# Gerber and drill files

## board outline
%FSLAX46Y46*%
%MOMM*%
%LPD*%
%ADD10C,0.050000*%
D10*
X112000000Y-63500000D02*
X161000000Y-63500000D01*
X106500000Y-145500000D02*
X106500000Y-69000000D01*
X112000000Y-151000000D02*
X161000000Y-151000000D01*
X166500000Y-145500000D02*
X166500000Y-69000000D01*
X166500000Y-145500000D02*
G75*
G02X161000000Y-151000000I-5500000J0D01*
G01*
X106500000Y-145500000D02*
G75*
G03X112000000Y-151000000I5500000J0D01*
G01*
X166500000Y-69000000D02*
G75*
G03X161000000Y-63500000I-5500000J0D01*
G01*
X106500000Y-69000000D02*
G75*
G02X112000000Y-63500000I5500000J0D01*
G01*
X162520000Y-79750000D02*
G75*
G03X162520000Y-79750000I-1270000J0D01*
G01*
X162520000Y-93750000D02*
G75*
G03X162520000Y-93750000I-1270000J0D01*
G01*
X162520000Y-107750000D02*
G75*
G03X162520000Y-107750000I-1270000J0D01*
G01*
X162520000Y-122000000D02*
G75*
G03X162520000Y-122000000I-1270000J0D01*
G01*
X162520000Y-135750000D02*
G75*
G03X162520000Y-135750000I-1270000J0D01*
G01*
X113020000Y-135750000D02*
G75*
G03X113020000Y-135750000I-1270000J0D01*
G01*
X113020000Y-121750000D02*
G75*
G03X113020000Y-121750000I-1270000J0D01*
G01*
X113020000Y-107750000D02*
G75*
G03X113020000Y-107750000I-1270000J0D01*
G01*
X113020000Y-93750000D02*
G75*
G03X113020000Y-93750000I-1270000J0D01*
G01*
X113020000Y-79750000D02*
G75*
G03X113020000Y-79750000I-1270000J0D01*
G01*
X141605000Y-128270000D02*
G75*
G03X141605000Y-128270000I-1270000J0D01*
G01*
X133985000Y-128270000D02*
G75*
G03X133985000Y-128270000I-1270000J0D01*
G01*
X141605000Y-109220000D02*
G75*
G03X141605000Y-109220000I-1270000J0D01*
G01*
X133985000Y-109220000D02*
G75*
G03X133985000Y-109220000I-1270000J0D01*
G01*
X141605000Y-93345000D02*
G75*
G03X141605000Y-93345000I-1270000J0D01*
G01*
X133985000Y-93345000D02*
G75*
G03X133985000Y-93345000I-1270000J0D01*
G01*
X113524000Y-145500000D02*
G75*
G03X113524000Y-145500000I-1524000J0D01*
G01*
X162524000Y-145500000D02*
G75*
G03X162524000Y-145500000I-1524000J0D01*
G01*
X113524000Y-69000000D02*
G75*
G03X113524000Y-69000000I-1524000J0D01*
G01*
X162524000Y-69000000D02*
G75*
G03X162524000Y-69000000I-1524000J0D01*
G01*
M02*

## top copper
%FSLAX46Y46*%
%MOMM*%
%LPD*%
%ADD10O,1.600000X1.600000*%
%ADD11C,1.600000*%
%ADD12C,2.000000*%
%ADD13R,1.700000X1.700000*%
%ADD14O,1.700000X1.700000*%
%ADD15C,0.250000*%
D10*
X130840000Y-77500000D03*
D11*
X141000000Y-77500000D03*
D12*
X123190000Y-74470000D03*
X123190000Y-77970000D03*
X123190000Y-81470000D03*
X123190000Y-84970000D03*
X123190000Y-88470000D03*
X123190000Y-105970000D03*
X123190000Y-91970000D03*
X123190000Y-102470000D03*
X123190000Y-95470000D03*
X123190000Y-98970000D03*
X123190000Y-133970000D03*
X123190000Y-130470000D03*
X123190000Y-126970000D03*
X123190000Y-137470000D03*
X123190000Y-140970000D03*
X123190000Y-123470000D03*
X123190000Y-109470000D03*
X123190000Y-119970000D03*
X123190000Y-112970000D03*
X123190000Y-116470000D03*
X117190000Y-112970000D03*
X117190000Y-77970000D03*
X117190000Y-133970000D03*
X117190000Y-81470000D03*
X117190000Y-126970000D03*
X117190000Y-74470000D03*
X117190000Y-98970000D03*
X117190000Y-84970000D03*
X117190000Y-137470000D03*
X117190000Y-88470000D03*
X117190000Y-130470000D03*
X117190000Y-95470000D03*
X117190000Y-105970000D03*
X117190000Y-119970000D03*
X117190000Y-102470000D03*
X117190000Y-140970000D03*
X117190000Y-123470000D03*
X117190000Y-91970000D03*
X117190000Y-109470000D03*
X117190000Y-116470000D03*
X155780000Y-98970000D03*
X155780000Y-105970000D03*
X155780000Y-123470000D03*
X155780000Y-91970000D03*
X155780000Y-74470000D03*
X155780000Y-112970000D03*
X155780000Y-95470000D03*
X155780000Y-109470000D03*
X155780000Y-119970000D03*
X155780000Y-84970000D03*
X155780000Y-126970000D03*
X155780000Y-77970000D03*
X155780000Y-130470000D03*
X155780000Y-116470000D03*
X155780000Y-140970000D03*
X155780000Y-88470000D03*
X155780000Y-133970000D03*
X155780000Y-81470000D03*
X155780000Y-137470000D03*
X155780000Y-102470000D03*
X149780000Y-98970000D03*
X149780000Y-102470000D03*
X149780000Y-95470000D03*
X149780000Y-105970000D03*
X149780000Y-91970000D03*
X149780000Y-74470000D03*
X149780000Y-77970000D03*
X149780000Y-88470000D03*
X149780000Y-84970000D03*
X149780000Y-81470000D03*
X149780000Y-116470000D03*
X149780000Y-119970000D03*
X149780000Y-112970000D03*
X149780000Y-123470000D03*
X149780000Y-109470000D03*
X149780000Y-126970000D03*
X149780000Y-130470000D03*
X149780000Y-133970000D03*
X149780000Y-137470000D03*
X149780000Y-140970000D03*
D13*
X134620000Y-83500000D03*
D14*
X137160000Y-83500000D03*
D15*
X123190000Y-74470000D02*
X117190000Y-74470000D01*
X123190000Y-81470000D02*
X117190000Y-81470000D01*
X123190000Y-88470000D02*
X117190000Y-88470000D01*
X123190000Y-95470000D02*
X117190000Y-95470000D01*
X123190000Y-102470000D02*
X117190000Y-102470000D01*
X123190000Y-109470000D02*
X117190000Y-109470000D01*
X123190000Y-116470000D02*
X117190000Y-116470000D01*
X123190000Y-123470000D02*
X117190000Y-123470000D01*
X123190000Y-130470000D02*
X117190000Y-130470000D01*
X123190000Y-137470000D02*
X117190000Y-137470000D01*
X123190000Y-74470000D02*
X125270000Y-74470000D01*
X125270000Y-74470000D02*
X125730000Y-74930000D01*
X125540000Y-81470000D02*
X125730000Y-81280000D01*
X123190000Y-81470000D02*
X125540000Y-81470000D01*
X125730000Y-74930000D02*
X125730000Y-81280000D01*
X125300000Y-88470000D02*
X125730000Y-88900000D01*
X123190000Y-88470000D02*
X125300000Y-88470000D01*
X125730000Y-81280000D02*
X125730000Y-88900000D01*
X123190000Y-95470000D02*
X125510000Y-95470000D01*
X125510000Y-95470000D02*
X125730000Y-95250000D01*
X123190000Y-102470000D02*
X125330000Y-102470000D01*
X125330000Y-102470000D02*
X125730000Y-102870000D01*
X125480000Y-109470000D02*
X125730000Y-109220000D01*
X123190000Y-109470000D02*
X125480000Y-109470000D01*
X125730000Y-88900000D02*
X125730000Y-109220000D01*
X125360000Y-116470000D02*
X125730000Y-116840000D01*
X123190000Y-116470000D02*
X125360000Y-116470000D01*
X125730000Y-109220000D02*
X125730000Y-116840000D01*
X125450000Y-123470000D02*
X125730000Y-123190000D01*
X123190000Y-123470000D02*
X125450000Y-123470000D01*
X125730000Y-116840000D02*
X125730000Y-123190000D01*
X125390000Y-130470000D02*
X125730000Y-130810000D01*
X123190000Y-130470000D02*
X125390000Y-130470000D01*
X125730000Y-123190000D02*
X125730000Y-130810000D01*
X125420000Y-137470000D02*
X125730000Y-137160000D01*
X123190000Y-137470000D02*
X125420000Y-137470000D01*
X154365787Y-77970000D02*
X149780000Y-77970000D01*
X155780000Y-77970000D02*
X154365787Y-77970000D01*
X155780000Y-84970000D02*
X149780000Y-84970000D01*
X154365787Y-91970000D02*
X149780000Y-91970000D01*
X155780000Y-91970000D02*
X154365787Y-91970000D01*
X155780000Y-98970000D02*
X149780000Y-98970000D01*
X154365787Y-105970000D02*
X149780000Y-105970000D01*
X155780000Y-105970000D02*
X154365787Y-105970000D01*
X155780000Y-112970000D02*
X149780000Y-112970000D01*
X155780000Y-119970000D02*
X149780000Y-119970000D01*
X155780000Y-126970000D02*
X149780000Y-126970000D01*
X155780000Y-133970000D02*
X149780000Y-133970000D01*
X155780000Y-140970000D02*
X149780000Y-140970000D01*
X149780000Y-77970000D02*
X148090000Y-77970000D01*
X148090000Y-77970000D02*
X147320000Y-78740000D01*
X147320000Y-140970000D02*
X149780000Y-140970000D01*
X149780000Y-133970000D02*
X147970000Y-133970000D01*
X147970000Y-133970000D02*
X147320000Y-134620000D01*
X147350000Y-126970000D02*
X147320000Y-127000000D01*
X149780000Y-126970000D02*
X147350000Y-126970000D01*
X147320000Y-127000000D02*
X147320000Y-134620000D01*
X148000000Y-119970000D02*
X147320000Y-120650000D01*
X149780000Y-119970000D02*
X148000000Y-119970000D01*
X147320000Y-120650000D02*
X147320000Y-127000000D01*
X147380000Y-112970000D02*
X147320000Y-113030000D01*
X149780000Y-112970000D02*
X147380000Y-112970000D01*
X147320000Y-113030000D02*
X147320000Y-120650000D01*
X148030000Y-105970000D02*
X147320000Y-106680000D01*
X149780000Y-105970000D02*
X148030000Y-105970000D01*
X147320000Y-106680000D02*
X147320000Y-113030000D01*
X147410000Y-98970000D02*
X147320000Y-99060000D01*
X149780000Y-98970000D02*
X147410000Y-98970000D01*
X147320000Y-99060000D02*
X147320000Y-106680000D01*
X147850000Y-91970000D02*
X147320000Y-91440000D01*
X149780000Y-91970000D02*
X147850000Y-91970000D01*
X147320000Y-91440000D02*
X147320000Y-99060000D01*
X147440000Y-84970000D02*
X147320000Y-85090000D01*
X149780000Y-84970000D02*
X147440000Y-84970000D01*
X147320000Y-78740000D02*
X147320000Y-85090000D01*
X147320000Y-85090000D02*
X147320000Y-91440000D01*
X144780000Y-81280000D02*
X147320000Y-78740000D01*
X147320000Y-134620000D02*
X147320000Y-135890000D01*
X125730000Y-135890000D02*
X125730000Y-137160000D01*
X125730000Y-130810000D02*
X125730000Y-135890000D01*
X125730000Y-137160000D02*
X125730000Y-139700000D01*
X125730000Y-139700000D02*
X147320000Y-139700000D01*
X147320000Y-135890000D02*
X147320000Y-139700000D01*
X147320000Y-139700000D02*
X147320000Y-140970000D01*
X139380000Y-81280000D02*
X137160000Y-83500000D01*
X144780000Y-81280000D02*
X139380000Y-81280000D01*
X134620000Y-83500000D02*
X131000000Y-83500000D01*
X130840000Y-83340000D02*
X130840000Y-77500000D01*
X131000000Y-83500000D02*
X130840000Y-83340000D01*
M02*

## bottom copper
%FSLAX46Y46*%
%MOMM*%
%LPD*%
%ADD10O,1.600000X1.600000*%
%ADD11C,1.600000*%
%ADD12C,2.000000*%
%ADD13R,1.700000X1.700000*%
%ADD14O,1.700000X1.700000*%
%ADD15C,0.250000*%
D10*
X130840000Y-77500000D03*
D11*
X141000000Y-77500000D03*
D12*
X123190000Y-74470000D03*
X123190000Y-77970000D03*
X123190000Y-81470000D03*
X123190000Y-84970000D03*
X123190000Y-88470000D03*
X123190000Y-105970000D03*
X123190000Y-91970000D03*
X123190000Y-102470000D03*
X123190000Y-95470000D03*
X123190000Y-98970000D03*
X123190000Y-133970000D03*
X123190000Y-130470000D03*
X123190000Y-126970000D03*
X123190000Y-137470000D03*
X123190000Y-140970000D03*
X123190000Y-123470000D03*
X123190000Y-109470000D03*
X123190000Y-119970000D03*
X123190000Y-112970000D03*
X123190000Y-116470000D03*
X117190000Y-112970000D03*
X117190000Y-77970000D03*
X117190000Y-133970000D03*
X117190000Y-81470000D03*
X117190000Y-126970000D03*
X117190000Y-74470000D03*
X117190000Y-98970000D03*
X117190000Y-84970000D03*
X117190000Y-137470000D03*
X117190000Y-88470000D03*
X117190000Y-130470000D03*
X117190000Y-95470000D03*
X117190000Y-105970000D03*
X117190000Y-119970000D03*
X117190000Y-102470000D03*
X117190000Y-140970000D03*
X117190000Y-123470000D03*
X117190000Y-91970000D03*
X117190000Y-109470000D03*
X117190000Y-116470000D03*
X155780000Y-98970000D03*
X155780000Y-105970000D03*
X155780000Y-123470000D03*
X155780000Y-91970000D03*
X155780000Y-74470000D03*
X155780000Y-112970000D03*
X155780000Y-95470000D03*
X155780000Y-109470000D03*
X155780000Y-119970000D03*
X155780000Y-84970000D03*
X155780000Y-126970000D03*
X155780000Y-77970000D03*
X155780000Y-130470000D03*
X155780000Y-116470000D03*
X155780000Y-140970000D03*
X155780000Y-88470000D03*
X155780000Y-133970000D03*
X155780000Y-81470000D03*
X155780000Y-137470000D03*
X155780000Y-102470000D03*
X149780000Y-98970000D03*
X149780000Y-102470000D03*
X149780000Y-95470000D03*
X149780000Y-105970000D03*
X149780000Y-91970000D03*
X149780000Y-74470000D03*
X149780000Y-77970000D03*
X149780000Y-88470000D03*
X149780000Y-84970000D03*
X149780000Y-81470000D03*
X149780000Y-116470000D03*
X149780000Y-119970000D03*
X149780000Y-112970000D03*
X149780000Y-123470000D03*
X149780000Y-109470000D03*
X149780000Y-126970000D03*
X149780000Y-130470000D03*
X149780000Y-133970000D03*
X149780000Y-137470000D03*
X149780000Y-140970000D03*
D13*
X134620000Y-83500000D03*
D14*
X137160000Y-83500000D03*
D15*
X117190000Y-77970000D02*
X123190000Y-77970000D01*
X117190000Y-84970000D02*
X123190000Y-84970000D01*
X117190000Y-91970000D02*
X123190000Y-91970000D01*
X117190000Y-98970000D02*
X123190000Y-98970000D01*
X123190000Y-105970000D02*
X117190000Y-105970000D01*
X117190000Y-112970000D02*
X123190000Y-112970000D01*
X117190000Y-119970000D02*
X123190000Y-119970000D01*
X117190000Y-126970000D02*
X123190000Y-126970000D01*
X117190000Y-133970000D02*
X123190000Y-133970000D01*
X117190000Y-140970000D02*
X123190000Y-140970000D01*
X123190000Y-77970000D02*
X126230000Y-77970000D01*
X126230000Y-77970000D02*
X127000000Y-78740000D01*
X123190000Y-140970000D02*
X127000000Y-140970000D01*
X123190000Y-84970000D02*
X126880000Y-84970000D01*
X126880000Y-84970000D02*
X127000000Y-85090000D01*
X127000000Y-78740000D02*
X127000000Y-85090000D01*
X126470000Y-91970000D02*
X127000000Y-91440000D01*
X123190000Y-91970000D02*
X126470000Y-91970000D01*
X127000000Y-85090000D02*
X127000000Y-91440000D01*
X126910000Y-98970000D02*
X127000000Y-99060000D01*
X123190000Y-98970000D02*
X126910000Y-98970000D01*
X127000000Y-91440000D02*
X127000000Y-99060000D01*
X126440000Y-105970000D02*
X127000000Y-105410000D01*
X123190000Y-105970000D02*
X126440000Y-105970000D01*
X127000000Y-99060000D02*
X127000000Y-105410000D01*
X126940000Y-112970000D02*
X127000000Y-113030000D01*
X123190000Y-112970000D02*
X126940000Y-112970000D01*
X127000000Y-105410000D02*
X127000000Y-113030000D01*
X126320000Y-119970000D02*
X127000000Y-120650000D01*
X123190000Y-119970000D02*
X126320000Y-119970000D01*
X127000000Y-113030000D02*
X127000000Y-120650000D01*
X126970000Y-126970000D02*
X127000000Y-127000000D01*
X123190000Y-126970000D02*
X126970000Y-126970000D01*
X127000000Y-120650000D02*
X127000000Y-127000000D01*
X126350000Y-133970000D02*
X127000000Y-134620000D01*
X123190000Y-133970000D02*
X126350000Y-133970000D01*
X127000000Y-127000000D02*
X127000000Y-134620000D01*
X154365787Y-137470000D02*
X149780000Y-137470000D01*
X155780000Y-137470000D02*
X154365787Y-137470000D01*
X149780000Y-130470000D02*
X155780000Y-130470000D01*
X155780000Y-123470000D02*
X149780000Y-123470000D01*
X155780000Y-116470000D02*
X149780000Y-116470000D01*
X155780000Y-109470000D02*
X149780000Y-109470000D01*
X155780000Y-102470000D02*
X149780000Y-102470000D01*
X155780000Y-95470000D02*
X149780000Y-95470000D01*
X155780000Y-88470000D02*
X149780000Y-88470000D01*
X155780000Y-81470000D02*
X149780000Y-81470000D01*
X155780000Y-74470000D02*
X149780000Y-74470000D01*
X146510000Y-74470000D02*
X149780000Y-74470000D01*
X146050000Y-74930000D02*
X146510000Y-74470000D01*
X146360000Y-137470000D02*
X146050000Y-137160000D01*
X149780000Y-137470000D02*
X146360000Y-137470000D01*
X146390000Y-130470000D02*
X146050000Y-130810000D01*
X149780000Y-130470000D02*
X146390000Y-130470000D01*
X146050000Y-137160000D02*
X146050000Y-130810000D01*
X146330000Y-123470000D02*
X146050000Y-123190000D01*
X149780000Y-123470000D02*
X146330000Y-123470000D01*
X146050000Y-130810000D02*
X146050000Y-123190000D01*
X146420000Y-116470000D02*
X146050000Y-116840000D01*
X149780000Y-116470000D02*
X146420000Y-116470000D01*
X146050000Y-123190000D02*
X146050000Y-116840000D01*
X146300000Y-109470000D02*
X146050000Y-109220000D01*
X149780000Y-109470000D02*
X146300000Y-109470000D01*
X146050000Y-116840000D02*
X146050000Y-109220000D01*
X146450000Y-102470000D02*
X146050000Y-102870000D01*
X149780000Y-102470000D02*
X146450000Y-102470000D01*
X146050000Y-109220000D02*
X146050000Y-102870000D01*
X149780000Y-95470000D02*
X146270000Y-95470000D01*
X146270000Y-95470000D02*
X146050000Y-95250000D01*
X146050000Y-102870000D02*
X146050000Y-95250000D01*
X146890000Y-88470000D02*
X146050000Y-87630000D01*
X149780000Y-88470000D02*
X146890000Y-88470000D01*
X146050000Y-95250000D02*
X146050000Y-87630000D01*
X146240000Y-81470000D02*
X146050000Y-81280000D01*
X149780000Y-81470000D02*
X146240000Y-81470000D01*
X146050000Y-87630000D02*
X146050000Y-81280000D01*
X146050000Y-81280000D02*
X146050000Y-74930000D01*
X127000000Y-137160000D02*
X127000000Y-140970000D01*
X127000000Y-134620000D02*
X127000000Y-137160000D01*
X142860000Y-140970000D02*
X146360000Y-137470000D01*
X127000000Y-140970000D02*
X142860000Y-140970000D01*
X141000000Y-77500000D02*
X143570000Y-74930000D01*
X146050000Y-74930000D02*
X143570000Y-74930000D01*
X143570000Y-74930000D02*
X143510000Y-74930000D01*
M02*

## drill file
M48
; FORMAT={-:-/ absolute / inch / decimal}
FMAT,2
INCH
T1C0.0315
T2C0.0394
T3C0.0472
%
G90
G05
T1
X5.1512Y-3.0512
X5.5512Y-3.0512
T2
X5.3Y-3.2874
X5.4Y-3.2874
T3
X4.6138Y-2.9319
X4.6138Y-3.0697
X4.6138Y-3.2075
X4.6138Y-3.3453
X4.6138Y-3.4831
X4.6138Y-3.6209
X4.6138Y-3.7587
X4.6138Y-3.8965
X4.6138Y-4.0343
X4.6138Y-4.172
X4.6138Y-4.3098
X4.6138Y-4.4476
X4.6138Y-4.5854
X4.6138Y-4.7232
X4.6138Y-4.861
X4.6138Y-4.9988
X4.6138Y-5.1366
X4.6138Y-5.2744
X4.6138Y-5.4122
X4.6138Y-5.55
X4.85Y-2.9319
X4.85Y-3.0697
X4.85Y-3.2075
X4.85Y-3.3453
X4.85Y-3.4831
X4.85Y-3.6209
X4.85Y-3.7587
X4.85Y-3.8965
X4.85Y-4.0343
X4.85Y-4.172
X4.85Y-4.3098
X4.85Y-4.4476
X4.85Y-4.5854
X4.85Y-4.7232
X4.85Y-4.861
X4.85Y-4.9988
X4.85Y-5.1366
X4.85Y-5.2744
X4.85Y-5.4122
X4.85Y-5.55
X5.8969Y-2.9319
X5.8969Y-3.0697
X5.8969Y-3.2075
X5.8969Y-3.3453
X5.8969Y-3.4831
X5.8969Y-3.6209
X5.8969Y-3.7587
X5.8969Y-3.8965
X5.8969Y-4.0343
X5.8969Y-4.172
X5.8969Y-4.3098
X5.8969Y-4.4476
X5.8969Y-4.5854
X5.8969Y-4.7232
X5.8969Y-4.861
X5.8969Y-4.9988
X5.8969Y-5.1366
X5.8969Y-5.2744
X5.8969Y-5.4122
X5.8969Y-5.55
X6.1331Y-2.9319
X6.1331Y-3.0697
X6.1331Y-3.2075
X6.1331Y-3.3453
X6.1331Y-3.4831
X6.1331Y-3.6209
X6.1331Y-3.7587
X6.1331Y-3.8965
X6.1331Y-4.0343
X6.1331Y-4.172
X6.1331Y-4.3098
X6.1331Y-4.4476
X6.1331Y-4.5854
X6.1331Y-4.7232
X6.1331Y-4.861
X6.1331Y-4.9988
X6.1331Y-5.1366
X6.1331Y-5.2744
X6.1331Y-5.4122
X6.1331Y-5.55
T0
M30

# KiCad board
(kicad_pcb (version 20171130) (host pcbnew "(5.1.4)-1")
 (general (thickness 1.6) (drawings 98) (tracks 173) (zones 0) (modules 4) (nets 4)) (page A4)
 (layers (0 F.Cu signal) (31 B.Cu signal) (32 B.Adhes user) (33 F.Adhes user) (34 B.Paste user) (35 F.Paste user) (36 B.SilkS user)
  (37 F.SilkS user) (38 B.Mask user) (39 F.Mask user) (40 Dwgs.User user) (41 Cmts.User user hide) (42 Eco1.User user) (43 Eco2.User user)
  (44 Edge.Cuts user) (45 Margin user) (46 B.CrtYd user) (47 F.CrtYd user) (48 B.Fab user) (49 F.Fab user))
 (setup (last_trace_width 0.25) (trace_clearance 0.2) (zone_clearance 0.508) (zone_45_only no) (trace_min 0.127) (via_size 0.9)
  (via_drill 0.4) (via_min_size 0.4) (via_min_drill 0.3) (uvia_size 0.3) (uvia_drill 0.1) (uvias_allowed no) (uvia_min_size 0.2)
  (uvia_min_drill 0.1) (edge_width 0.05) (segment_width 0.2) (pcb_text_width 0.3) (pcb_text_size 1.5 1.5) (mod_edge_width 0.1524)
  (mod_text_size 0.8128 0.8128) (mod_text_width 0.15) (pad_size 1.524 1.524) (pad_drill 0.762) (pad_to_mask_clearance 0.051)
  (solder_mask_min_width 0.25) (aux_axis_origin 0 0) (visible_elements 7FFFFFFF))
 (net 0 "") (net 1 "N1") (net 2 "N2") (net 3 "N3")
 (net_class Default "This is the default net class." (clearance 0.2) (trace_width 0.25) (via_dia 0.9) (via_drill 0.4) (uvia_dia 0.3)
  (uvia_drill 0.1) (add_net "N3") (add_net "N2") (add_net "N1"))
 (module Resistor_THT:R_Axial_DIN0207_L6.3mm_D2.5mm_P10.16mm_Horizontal (layer F.Cu) (at 141 77.5 180)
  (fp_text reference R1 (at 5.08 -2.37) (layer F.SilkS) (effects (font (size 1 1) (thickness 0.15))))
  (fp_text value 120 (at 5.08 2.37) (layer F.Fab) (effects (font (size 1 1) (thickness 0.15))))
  (pad 2 thru_hole oval (at 10.16 0 180) (size 1.6 1.6) (drill 0.8) (layers *.Cu *.Mask) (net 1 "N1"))
  (pad 1 thru_hole circle (at 0 0 180) (size 1.6 1.6) (drill 0.8) (layers *.Cu *.Mask) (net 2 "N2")))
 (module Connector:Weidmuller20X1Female (layer F.Cu) (at 128.19 88.97 270)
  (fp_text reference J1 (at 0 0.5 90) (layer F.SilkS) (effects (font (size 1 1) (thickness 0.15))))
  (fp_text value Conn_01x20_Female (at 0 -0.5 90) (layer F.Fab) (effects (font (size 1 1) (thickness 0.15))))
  (pad 1 thru_hole circle (at -14.5 5 270) (size 2 2) (drill 1.2) (layers *.Cu *.Mask) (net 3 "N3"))
  (pad 2 thru_hole circle (at -11 5 270) (size 2 2) (drill 1.2) (layers *.Cu *.Mask) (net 2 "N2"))
  (pad 3 thru_hole circle (at -7.5 5 270) (size 2 2) (drill 1.2) (layers *.Cu *.Mask) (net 3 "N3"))
  (pad 4 thru_hole circle (at -4 5) (size 2 2) (drill 1.2) (layers *.Cu *.Mask) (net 2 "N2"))
  (pad 5 thru_hole circle (at -0.5 5 270) (size 2 2) (drill 1.2) (layers *.Cu *.Mask) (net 3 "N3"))
  (pad 10 thru_hole circle (at 17 5 270) (size 2 2) (drill 1.2) (layers *.Cu *.Mask) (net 2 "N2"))
  (pad 6 thru_hole circle (at 3 5 270) (size 2 2) (drill 1.2) (layers *.Cu *.Mask) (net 2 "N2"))
  (pad 9 thru_hole circle (at 13.5 5 270) (size 2 2) (drill 1.2) (layers *.Cu *.Mask) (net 3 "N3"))
  (pad 7 thru_hole circle (at 6.5 5 270) (size 2 2) (drill 1.2) (layers *.Cu *.Mask) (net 3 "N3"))
  (pad 8 thru_hole circle (at 10 5 270) (size 2 2) (drill 1.2) (layers *.Cu *.Mask) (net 2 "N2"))
  (pad 18 thru_hole circle (at 45 5 270) (size 2 2) (drill 1.2) (layers *.Cu *.Mask) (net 2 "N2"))
  (pad 17 thru_hole circle (at 41.5 5) (size 2 2) (drill 1.2) (layers *.Cu *.Mask) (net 3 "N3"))
  (pad 16 thru_hole circle (at 38 5 270) (size 2 2) (drill 1.2) (layers *.Cu *.Mask) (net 2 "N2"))
  (pad 19 thru_hole circle (at 48.5 5 270) (size 2 2) (drill 1.2) (layers *.Cu *.Mask) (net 3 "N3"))
  (pad 20 thru_hole circle (at 52 5 270) (size 2 2) (drill 1.2) (layers *.Cu *.Mask) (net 2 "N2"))
  (pad 15 thru_hole circle (at 34.5 5 270) (size 2 2) (drill 1.2) (layers *.Cu *.Mask) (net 3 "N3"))
  (pad 11 thru_hole circle (at 20.5 5 270) (size 2 2) (drill 1.2) (layers *.Cu *.Mask) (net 3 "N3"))
  (pad 14 thru_hole circle (at 31 5 270) (size 2 2) (drill 1.2) (layers *.Cu *.Mask) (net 2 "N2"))
  (pad 12 thru_hole circle (at 24 5 270) (size 2 2) (drill 1.2) (layers *.Cu *.Mask) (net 2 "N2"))
  (pad 13 thru_hole circle (at 27.5 5 270) (size 2 2) (drill 1.2) (layers *.Cu *.Mask) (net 3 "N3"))
  (pad 12 thru_hole circle (at 24 11 270) (size 2 2) (drill 1.2) (layers *.Cu *.Mask) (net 2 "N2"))
  (pad 2 thru_hole circle (at -11 11 270) (size 2 2) (drill 1.2) (layers *.Cu *.Mask) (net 2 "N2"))
  (pad 18 thru_hole circle (at 45 11 270) (size 2 2) (drill 1.2) (layers *.Cu *.Mask) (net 2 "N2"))
  (pad 3 thru_hole circle (at -7.5 11 270) (size 2 2) (drill 1.2) (layers *.Cu *.Mask) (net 3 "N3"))
  (pad 16 thru_hole circle (at 38 11 270) (size 2 2) (drill 1.2) (layers *.Cu *.Mask) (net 2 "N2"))
  (pad 1 thru_hole circle (at -14.5 11 270) (size 2 2) (drill 1.2) (layers *.Cu *.Mask) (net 3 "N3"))
  (pad 8 thru_hole circle (at 10 11 270) (size 2 2) (drill 1.2) (layers *.Cu *.Mask) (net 2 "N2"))
  (pad 4 thru_hole circle (at -4 11) (size 2 2) (drill 1.2) (layers *.Cu *.Mask) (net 2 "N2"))
  (pad 19 thru_hole circle (at 48.5 11 270) (size 2 2) (drill 1.2) (layers *.Cu *.Mask) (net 3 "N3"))
  (pad 5 thru_hole circle (at -0.5 11 270) (size 2 2) (drill 1.2) (layers *.Cu *.Mask) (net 3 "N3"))
  (pad 17 thru_hole circle (at 41.5 11) (size 2 2) (drill 1.2) (layers *.Cu *.Mask) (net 3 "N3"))
  (pad 7 thru_hole circle (at 6.5 11 270) (size 2 2) (drill 1.2) (layers *.Cu *.Mask) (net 3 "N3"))
  (pad 10 thru_hole circle (at 17 11 270) (size 2 2) (drill 1.2) (layers *.Cu *.Mask) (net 2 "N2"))
  (pad 14 thru_hole circle (at 31 11 270) (size 2 2) (drill 1.2) (layers *.Cu *.Mask) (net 2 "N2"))
  (pad 9 thru_hole circle (at 13.5 11 270) (size 2 2) (drill 1.2) (layers *.Cu *.Mask) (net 3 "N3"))
  (pad 20 thru_hole circle (at 52 11 270) (size 2 2) (drill 1.2) (layers *.Cu *.Mask) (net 2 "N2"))
  (pad 15 thru_hole circle (at 34.5 11 270) (size 2 2) (drill 1.2) (layers *.Cu *.Mask) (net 3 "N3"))
  (pad 6 thru_hole circle (at 3 11 270) (size 2 2) (drill 1.2) (layers *.Cu *.Mask) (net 2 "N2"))
  (pad 11 thru_hole circle (at 20.5 11 270) (size 2 2) (drill 1.2) (layers *.Cu *.Mask) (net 3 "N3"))
  (pad 13 thru_hole circle (at 27.5 11 270) (size 2 2) (drill 1.2) (layers *.Cu *.Mask) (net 3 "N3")))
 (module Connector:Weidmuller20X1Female (layer F.Cu) (at 144.78 126.47 90)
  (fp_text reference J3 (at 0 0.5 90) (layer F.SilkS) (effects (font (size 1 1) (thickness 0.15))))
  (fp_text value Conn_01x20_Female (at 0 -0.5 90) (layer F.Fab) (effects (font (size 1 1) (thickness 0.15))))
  (pad 13 thru_hole circle (at 27.5 11 90) (size 2 2) (drill 1.2) (layers *.Cu *.Mask) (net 3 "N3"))
  (pad 11 thru_hole circle (at 20.5 11 90) (size 2 2) (drill 1.2) (layers *.Cu *.Mask) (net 3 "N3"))
  (pad 6 thru_hole circle (at 3 11 90) (size 2 2) (drill 1.2) (layers *.Cu *.Mask) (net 2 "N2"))
  (pad 15 thru_hole circle (at 34.5 11 90) (size 2 2) (drill 1.2) (layers *.Cu *.Mask) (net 3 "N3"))
  (pad 20 thru_hole circle (at 52 11 90) (size 2 2) (drill 1.2) (layers *.Cu *.Mask) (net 2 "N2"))
  (pad 9 thru_hole circle (at 13.5 11 90) (size 2 2) (drill 1.2) (layers *.Cu *.Mask) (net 3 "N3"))
  (pad 14 thru_hole circle (at 31 11 90) (size 2 2) (drill 1.2) (layers *.Cu *.Mask) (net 2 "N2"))
  (pad 10 thru_hole circle (at 17 11 90) (size 2 2) (drill 1.2) (layers *.Cu *.Mask) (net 2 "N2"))
  (pad 7 thru_hole circle (at 6.5 11 90) (size 2 2) (drill 1.2) (layers *.Cu *.Mask) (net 3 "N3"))
  (pad 17 thru_hole circle (at 41.5 11 180) (size 2 2) (drill 1.2) (layers *.Cu *.Mask) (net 3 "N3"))
  (pad 5 thru_hole circle (at -0.5 11 90) (size 2 2) (drill 1.2) (layers *.Cu *.Mask) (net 3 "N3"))
  (pad 19 thru_hole circle (at 48.5 11 90) (size 2 2) (drill 1.2) (layers *.Cu *.Mask) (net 3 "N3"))
  (pad 4 thru_hole circle (at -4 11 180) (size 2 2) (drill 1.2) (layers *.Cu *.Mask) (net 2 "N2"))
  (pad 8 thru_hole circle (at 10 11 90) (size 2 2) (drill 1.2) (layers *.Cu *.Mask) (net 2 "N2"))
  (pad 1 thru_hole circle (at -14.5 11 90) (size 2 2) (drill 1.2) (layers *.Cu *.Mask) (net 3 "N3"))
  (pad 16 thru_hole circle (at 38 11 90) (size 2 2) (drill 1.2) (layers *.Cu *.Mask) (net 2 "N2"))
  (pad 3 thru_hole circle (at -7.5 11 90) (size 2 2) (drill 1.2) (layers *.Cu *.Mask) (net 3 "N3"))
  (pad 18 thru_hole circle (at 45 11 90) (size 2 2) (drill 1.2) (layers *.Cu *.Mask) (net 2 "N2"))
  (pad 2 thru_hole circle (at -11 11 90) (size 2 2) (drill 1.2) (layers *.Cu *.Mask) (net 2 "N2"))
  (pad 12 thru_hole circle (at 24 11 90) (size 2 2) (drill 1.2) (layers *.Cu *.Mask) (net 2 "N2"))
  (pad 13 thru_hole circle (at 27.5 5 90) (size 2 2) (drill 1.2) (layers *.Cu *.Mask) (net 3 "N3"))
  (pad 12 thru_hole circle (at 24 5 90) (size 2 2) (drill 1.2) (layers *.Cu *.Mask) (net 2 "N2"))
  (pad 14 thru_hole circle (at 31 5 90) (size 2 2) (drill 1.2) (layers *.Cu *.Mask) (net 2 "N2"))
  (pad 11 thru_hole circle (at 20.5 5 90) (size 2 2) (drill 1.2) (layers *.Cu *.Mask) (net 3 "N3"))
  (pad 15 thru_hole circle (at 34.5 5 90) (size 2 2) (drill 1.2) (layers *.Cu *.Mask) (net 3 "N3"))
  (pad 20 thru_hole circle (at 52 5 90) (size 2 2) (drill 1.2) (layers *.Cu *.Mask) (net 2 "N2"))
  (pad 19 thru_hole circle (at 48.5 5 90) (size 2 2) (drill 1.2) (layers *.Cu *.Mask) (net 3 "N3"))
  (pad 16 thru_hole circle (at 38 5 90) (size 2 2) (drill 1.2) (layers *.Cu *.Mask) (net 2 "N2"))
  (pad 17 thru_hole circle (at 41.5 5 180) (size 2 2) (drill 1.2) (layers *.Cu *.Mask) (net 3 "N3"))
  (pad 18 thru_hole circle (at 45 5 90) (size 2 2) (drill 1.2) (layers *.Cu *.Mask) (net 2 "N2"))
  (pad 8 thru_hole circle (at 10 5 90) (size 2 2) (drill 1.2) (layers *.Cu *.Mask) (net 2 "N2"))
  (pad 7 thru_hole circle (at 6.5 5 90) (size 2 2) (drill 1.2) (layers *.Cu *.Mask) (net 3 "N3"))
  (pad 9 thru_hole circle (at 13.5 5 90) (size 2 2) (drill 1.2) (layers *.Cu *.Mask) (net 3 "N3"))
  (pad 6 thru_hole circle (at 3 5 90) (size 2 2) (drill 1.2) (layers *.Cu *.Mask) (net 2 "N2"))
  (pad 10 thru_hole circle (at 17 5 90) (size 2 2) (drill 1.2) (layers *.Cu *.Mask) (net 2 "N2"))
  (pad 5 thru_hole circle (at -0.5 5 90) (size 2 2) (drill 1.2) (layers *.Cu *.Mask) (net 3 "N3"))
  (pad 4 thru_hole circle (at -4 5 180) (size 2 2) (drill 1.2) (layers *.Cu *.Mask) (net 2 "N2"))
  (pad 3 thru_hole circle (at -7.5 5 90) (size 2 2) (drill 1.2) (layers *.Cu *.Mask) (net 3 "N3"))
  (pad 2 thru_hole circle (at -11 5 90) (size 2 2) (drill 1.2) (layers *.Cu *.Mask) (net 2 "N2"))
  (pad 1 thru_hole circle (at -14.5 5 90) (size 2 2) (drill 1.2) (layers *.Cu *.Mask) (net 3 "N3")))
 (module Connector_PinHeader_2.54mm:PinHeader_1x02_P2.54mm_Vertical (layer F.Cu) (at 134.62 83.5 90)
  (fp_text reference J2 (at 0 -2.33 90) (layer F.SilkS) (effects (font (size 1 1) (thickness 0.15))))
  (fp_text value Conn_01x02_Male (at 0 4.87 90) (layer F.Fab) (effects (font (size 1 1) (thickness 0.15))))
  (pad 1 thru_hole rect (at 0 0 90) (size 1.7 1.7) (drill 1) (layers *.Cu *.Mask) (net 1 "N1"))
  (pad 2 thru_hole oval (at 0 2.54 90) (size 1.7 1.7) (drill 1) (layers *.Cu *.Mask) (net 3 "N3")))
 (gr_line (start 112 63.5) (end 161 63.5) (layer Edge.Cuts) (width 0.05))
 (gr_line (start 106.5 145.5) (end 106.5 69) (layer Edge.Cuts) (width 0.05))
 (gr_line (start 112 151) (end 161 151) (layer Edge.Cuts) (width 0.05))
 (gr_line (start 166.5 145.5) (end 166.5 69) (layer Edge.Cuts) (width 0.05))
 (gr_arc (start 161 145.5) (end 161 151) (angle -90) (layer Edge.Cuts) (width 0.05))
 (gr_arc (start 112 145.5) (end 112 151) (angle 90) (layer Edge.Cuts) (width 0.05))
 (gr_arc (start 161 69) (end 161 63.5) (angle 90) (layer Edge.Cuts) (width 0.05))
 (gr_arc (start 112 69) (end 112 63.5) (angle -90) (layer Edge.Cuts) (width 0.05))
 (gr_circle (center 161.25 79.75) (end 162.52 79.75) (layer Edge.Cuts) (width 0.05))
 (gr_circle (center 161.25 93.75) (end 162.52 93.75) (layer Edge.Cuts) (width 0.05))
 (gr_circle (center 161.25 107.75) (end 162.52 107.75) (layer Edge.Cuts) (width 0.05))
 (gr_circle (center 161.25 122) (end 162.52 122) (layer Edge.Cuts) (width 0.05))
 (gr_circle (center 161.25 135.75) (end 162.52 135.75) (layer Edge.Cuts) (width 0.05))
 (gr_circle (center 111.75 135.75) (end 113.02 135.75) (layer Edge.Cuts) (width 0.05))
 (gr_circle (center 111.75 121.75) (end 113.02 121.75) (layer Edge.Cuts) (width 0.05))
 (gr_circle (center 111.75 107.75) (end 113.02 107.75) (layer Edge.Cuts) (width 0.05))
 (gr_circle (center 111.75 93.75) (end 113.02 93.75) (layer Edge.Cuts) (width 0.05))
 (gr_circle (center 111.75 79.75) (end 113.02 79.75) (layer Edge.Cuts) (width 0.05))
 (gr_circle (center 140.335 128.27) (end 140.335 127) (layer Edge.Cuts) (width 0.05))
 (gr_circle (center 132.715 128.27) (end 132.715 127) (layer Edge.Cuts) (width 0.05))
 (gr_circle (center 140.335 109.22) (end 140.335 107.95) (layer Edge.Cuts) (width 0.05))
 (gr_circle (center 132.715 109.22) (end 132.715 107.95) (layer Edge.Cuts) (width 0.05))
 (gr_circle (center 140.335 93.345) (end 140.335 92.075) (layer Edge.Cuts) (width 0.05))
 (gr_circle (center 132.715 93.345) (end 132.715 92.075) (layer Edge.Cuts) (width 0.05))
 (gr_circle (center 112 145.5) (end 113.524 145.5) (layer Edge.Cuts) (width 0.05))
 (gr_circle (center 161 145.5) (end 162.524 145.5) (layer Edge.Cuts) (width 0.05))
 (gr_circle (center 112 69) (end 113.524 69) (layer Edge.Cuts) (width 0.05))
 (gr_circle (center 161 69) (end 162.524 69) (layer Edge.Cuts) (width 0.05))
 (segment (start 123.19 74.47) (end 117.19 74.47) (width 0.25) (layer F.Cu) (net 3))
 (segment (start 123.19 81.47) (end 117.19 81.47) (width 0.25) (layer F.Cu) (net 3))
 (segment (start 123.19 88.47) (end 117.19 88.47) (width 0.25) (layer F.Cu) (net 3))
 (segment (start 123.19 95.47) (end 117.19 95.47) (width 0.25) (layer F.Cu) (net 3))
 (segment (start 123.19 102.47) (end 117.19 102.47) (width 0.25) (layer F.Cu) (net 3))
 (segment (start 123.19 109.47) (end 117.19 109.47) (width 0.25) (layer F.Cu) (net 3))
 (segment (start 123.19 116.47) (end 117.19 116.47) (width 0.25) (layer F.Cu) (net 3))
 (segment (start 123.19 123.47) (end 117.19 123.47) (width 0.25) (layer F.Cu) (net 3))
 (segment (start 123.19 130.47) (end 117.19 130.47) (width 0.25) (layer F.Cu) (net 3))
 (segment (start 123.19 137.47) (end 117.19 137.47) (width 0.25) (layer F.Cu) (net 3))
 (segment (start 123.19 74.47) (end 125.27 74.47) (width 0.25) (layer F.Cu) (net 3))
 (segment (start 125.27 74.47) (end 125.73 74.93) (width 0.25) (layer F.Cu) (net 3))
 (segment (start 125.54 81.47) (end 125.73 81.28) (width 0.25) (layer F.Cu) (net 3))
 (segment (start 123.19 81.47) (end 125.54 81.47) (width 0.25) (layer F.Cu) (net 3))
 (segment (start 125.73 74.93) (end 125.73 81.28) (width 0.25) (layer F.Cu) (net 3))
 (segment (start 125.3 88.47) (end 125.73 88.9) (width 0.25) (layer F.Cu) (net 3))
 (segment (start 123.19 88.47) (end 125.3 88.47) (width 0.25) (layer F.Cu) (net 3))
 (segment (start 125.73 81.28) (end 125.73 88.9) (width 0.25) (layer F.Cu) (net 3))
 (segment (start 123.19 95.47) (end 125.51 95.47) (width 0.25) (layer F.Cu) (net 3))
 (segment (start 125.51 95.47) (end 125.73 95.25) (width 0.25) (layer F.Cu) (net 3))
 (segment (start 123.19 102.47) (end 125.33 102.47) (width 0.25) (layer F.Cu) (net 3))
 (segment (start 125.33 102.47) (end 125.73 102.87) (width 0.25) (layer F.Cu) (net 3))
 (segment (start 125.48 109.47) (end 125.73 109.22) (width 0.25) (layer F.Cu) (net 3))
 (segment (start 123.19 109.47) (end 125.48 109.47) (width 0.25) (layer F.Cu) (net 3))
 (segment (start 125.73 88.9) (end 125.73 109.22) (width 0.25) (layer F.Cu) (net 3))
 (segment (start 125.36 116.47) (end 125.73 116.84) (width 0.25) (layer F.Cu) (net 3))
 (segment (start 123.19 116.47) (end 125.36 116.47) (width 0.25) (layer F.Cu) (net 3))
 (segment (start 125.73 109.22) (end 125.73 116.84) (width 0.25) (layer F.Cu) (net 3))
 (segment (start 125.45 123.47) (end 125.73 123.19) (width 0.25) (layer F.Cu) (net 3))
 (segment (start 123.19 123.47) (end 125.45 123.47) (width 0.25) (layer F.Cu) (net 3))
 (segment (start 125.73 116.84) (end 125.73 123.19) (width 0.25) (layer F.Cu) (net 3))
 (segment (start 125.39 130.47) (end 125.73 130.81) (width 0.25) (layer F.Cu) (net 3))
 (segment (start 123.19 130.47) (end 125.39 130.47) (width 0.25) (layer F.Cu) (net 3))
 (segment (start 125.73 123.19) (end 125.73 130.81) (width 0.25) (layer F.Cu) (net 3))
 (segment (start 125.42 137.47) (end 125.73 137.16) (width 0.25) (layer F.Cu) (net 3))
 (segment (start 123.19 137.47) (end 125.42 137.47) (width 0.25) (layer F.Cu) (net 3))
 (segment (start 154.365787 77.97) (end 149.78 77.97) (width 0.25) (layer F.Cu) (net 3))
 (segment (start 155.78 77.97) (end 154.365787 77.97) (width 0.25) (layer F.Cu) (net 3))
 (segment (start 155.78 84.97) (end 149.78 84.97) (width 0.25) (layer F.Cu) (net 3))
 (segment (start 154.365787 91.97) (end 149.78 91.97) (width 0.25) (layer F.Cu) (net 3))
 (segment (start 155.78 91.97) (end 154.365787 91.97) (width 0.25) (layer F.Cu) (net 3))
 (segment (start 155.78 98.97) (end 149.78 98.97) (width 0.25) (layer F.Cu) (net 3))
 (segment (start 154.365787 105.97) (end 149.78 105.97) (width 0.25) (layer F.Cu) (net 3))
 (segment (start 155.78 105.97) (end 154.365787 105.97) (width 0.25) (layer F.Cu) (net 3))
 (segment (start 155.78 112.97) (end 149.78 112.97) (width 0.25) (layer F.Cu) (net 3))
 (segment (start 155.78 119.97) (end 149.78 119.97) (width 0.25) (layer F.Cu) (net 3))
 (segment (start 155.78 126.97) (end 149.78 126.97) (width 0.25) (layer F.Cu) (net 3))
 (segment (start 155.78 133.97) (end 149.78 133.97) (width 0.25) (layer F.Cu) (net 3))
 (segment (start 155.78 140.97) (end 149.78 140.97) (width 0.25) (layer F.Cu) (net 3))
 (segment (start 149.78 77.97) (end 148.09 77.97) (width 0.25) (layer F.Cu) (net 3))
 (segment (start 148.09 77.97) (end 147.32 78.74) (width 0.25) (layer F.Cu) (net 3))
 (segment (start 147.32 140.97) (end 149.78 140.97) (width 0.25) (layer F.Cu) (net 3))
 (segment (start 149.78 133.97) (end 147.97 133.97) (width 0.25) (layer F.Cu) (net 3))
 (segment (start 147.97 133.97) (end 147.32 134.62) (width 0.25) (layer F.Cu) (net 3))
 (segment (start 147.35 126.97) (end 147.32 127) (width 0.25) (layer F.Cu) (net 3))
 (segment (start 149.78 126.97) (end 147.35 126.97) (width 0.25) (layer F.Cu) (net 3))
 (segment (start 147.32 127) (end 147.32 134.62) (width 0.25) (layer F.Cu) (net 3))
 (segment (start 148 119.97) (end 147.32 120.65) (width 0.25) (layer F.Cu) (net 3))
 (segment (start 149.78 119.97) (end 148 119.97) (width 0.25) (layer F.Cu) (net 3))
 (segment (start 147.32 120.65) (end 147.32 127) (width 0.25) (layer F.Cu) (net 3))
 (segment (start 147.38 112.97) (end 147.32 113.03) (width 0.25) (layer F.Cu) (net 3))
 (segment (start 149.78 112.97) (end 147.38 112.97) (width 0.25) (layer F.Cu) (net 3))
 (segment (start 147.32 113.03) (end 147.32 120.65) (width 0.25) (layer F.Cu) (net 3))
 (segment (start 148.03 105.97) (end 147.32 106.68) (width 0.25) (layer F.Cu) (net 3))
 (segment (start 149.78 105.97) (end 148.03 105.97) (width 0.25) (layer F.Cu) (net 3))
 (segment (start 147.32 106.68) (end 147.32 113.03) (width 0.25) (layer F.Cu) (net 3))
 (segment (start 147.41 98.97) (end 147.32 99.06) (width 0.25) (layer F.Cu) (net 3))
 (segment (start 149.78 98.97) (end 147.41 98.97) (width 0.25) (layer F.Cu) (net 3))
 (segment (start 147.32 99.06) (end 147.32 106.68) (width 0.25) (layer F.Cu) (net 3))
 (segment (start 147.85 91.97) (end 147.32 91.44) (width 0.25) (layer F.Cu) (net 3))
 (segment (start 149.78 91.97) (end 147.85 91.97) (width 0.25) (layer F.Cu) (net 3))
 (segment (start 147.32 91.44) (end 147.32 99.06) (width 0.25) (layer F.Cu) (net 3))
 (segment (start 147.44 84.97) (end 147.32 85.09) (width 0.25) (layer F.Cu) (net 3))
 (segment (start 149.78 84.97) (end 147.44 84.97) (width 0.25) (layer F.Cu) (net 3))
 (segment (start 147.32 78.74) (end 147.32 85.09) (width 0.25) (layer F.Cu) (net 3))
 (segment (start 147.32 85.09) (end 147.32 91.44) (width 0.25) (layer F.Cu) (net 3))
 (segment (start 144.78 81.28) (end 147.32 78.74) (width 0.25) (layer F.Cu) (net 3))
 (segment (start 147.32 134.62) (end 147.32 135.89) (width 0.25) (layer F.Cu) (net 3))
 (segment (start 125.73 135.89) (end 125.73 137.16) (width 0.25) (layer F.Cu) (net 3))
 (segment (start 125.73 130.81) (end 125.73 135.89) (width 0.25) (layer F.Cu) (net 3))
 (segment (start 125.73 137.16) (end 125.73 139.7) (width 0.25) (layer F.Cu) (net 3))
 (segment (start 125.73 139.7) (end 147.32 139.7) (width 0.25) (layer F.Cu) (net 3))
 (segment (start 147.32 135.89) (end 147.32 139.7) (width 0.25) (layer F.Cu) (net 3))
 (segment (start 147.32 139.7) (end 147.32 140.97) (width 0.25) (layer F.Cu) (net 3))
 (segment (start 139.38 81.28) (end 137.16 83.5) (width 0.25) (layer F.Cu) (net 3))
 (segment (start 144.78 81.28) (end 139.38 81.28) (width 0.25) (layer F.Cu) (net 3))
 (segment (start 117.19 77.97) (end 123.19 77.97) (width 0.25) (layer B.Cu) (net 2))
 (segment (start 117.19 84.97) (end 123.19 84.97) (width 0.25) (layer B.Cu) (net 2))
 (segment (start 117.19 91.97) (end 123.19 91.97) (width 0.25) (layer B.Cu) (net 2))
 (segment (start 117.19 98.97) (end 123.19 98.97) (width 0.25) (layer B.Cu) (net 2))
 (segment (start 123.19 105.97) (end 117.19 105.97) (width 0.25) (layer B.Cu) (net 2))
 (segment (start 117.19 112.97) (end 123.19 112.97) (width 0.25) (layer B.Cu) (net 2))
 (segment (start 117.19 119.97) (end 123.19 119.97) (width 0.25) (layer B.Cu) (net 2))
 (segment (start 117.19 126.97) (end 123.19 126.97) (width 0.25) (layer B.Cu) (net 2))
 (segment (start 117.19 133.97) (end 123.19 133.97) (width 0.25) (layer B.Cu) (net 2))
 (segment (start 117.19 140.97) (end 123.19 140.97) (width 0.25) (layer B.Cu) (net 2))
 (segment (start 123.19 77.97) (end 126.23 77.97) (width 0.25) (layer B.Cu) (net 2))
 (segment (start 126.23 77.97) (end 127 78.74) (width 0.25) (layer B.Cu) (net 2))
 (segment (start 123.19 140.97) (end 127 140.97) (width 0.25) (layer B.Cu) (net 2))
 (segment (start 123.19 84.97) (end 126.88 84.97) (width 0.25) (layer B.Cu) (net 2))
 (segment (start 126.88 84.97) (end 127 85.09) (width 0.25) (layer B.Cu) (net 2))
 (segment (start 127 78.74) (end 127 85.09) (width 0.25) (layer B.Cu) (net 2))
 (segment (start 126.47 91.97) (end 127 91.44) (width 0.25) (layer B.Cu) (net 2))
 (segment (start 123.19 91.97) (end 126.47 91.97) (width 0.25) (layer B.Cu) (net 2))
 (segment (start 127 85.09) (end 127 91.44) (width 0.25) (layer B.Cu) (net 2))
 (segment (start 126.91 98.97) (end 127 99.06) (width 0.25) (layer B.Cu) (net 2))
 (segment (start 123.19 98.97) (end 126.91 98.97) (width 0.25) (layer B.Cu) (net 2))
 (segment (start 127 91.44) (end 127 99.06) (width 0.25) (layer B.Cu) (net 2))
 (segment (start 126.44 105.97) (end 127 105.41) (width 0.25) (layer B.Cu) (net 2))
 (segment (start 123.19 105.97) (end 126.44 105.97) (width 0.25) (layer B.Cu) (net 2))
 (segment (start 127 99.06) (end 127 105.41) (width 0.25) (layer B.Cu) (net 2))
 (segment (start 126.94 112.97) (end 127 113.03) (width 0.25) (layer B.Cu) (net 2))
 (segment (start 123.19 112.97) (end 126.94 112.97) (width 0.25) (layer B.Cu) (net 2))
 (segment (start 127 105.41) (end 127 113.03) (width 0.25) (layer B.Cu) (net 2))
 (segment (start 126.32 119.97) (end 127 120.65) (width 0.25) (layer B.Cu) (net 2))
 (segment (start 123.19 119.97) (end 126.32 119.97) (width 0.25) (layer B.Cu) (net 2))
 (segment (start 127 113.03) (end 127 120.65) (width 0.25) (layer B.Cu) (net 2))
 (segment (start 126.97 126.97) (end 127 127) (width 0.25) (layer B.Cu) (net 2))
 (segment (start 123.19 126.97) (end 126.97 126.97) (width 0.25) (layer B.Cu) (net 2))
 (segment (start 127 120.65) (end 127 127) (width 0.25) (layer B.Cu) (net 2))
 (segment (start 126.35 133.97) (end 127 134.62) (width 0.25) (layer B.Cu) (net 2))
 (segment (start 123.19 133.97) (end 126.35 133.97) (width 0.25) (layer B.Cu) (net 2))
 (segment (start 127 127) (end 127 134.62) (width 0.25) (layer B.Cu) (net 2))
 (segment (start 154.365787 137.47) (end 149.78 137.47) (width 0.25) (layer B.Cu) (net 2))
 (segment (start 155.78 137.47) (end 154.365787 137.47) (width 0.25) (layer B.Cu) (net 2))
 (segment (start 149.78 130.47) (end 155.78 130.47) (width 0.25) (layer B.Cu) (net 2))
 (segment (start 155.78 123.47) (end 149.78 123.47) (width 0.25) (layer B.Cu) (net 2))
 (segment (start 155.78 116.47) (end 149.78 116.47) (width 0.25) (layer B.Cu) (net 2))
 (segment (start 155.78 109.47) (end 149.78 109.47) (width 0.25) (layer B.Cu) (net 2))
 (segment (start 155.78 102.47) (end 149.78 102.47) (width 0.25) (layer B.Cu) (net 2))
 (segment (start 155.78 95.47) (end 149.78 95.47) (width 0.25) (layer B.Cu) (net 2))
 (segment (start 155.78 88.47) (end 149.78 88.47) (width 0.25) (layer B.Cu) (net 2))
 (segment (start 155.78 81.47) (end 149.78 81.47) (width 0.25) (layer B.Cu) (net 2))
 (segment (start 155.78 74.47) (end 149.78 74.47) (width 0.25) (layer B.Cu) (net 2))
 (segment (start 146.51 74.47) (end 149.78 74.47) (width 0.25) (layer B.Cu) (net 2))
 (segment (start 146.05 74.93) (end 146.51 74.47) (width 0.25) (layer B.Cu) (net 2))
 (segment (start 146.36 137.47) (end 146.05 137.16) (width 0.25) (layer B.Cu) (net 2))
 (segment (start 149.78 137.47) (end 146.36 137.47) (width 0.25) (layer B.Cu) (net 2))
 (segment (start 146.39 130.47) (end 146.05 130.81) (width 0.25) (layer B.Cu) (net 2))
 (segment (start 149.78 130.47) (end 146.39 130.47) (width 0.25) (layer B.Cu) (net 2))
 (segment (start 146.05 137.16) (end 146.05 130.81) (width 0.25) (layer B.Cu) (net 2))
 (segment (start 146.33 123.47) (end 146.05 123.19) (width 0.25) (layer B.Cu) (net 2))
 (segment (start 149.78 123.47) (end 146.33 123.47) (width 0.25) (layer B.Cu) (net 2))
 (segment (start 146.05 130.81) (end 146.05 123.19) (width 0.25) (layer B.Cu) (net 2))
 (segment (start 146.42 116.47) (end 146.05 116.84) (width 0.25) (layer B.Cu) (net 2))
 (segment (start 149.78 116.47) (end 146.42 116.47) (width 0.25) (layer B.Cu) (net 2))
 (segment (start 146.05 123.19) (end 146.05 116.84) (width 0.25) (layer B.Cu) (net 2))
 (segment (start 146.3 109.47) (end 146.05 109.22) (width 0.25) (layer B.Cu) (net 2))
 (segment (start 149.78 109.47) (end 146.3 109.47) (width 0.25) (layer B.Cu) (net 2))
 (segment (start 146.05 116.84) (end 146.05 109.22) (width 0.25) (layer B.Cu) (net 2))
 (segment (start 146.45 102.47) (end 146.05 102.87) (width 0.25) (layer B.Cu) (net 2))
 (segment (start 149.78 102.47) (end 146.45 102.47) (width 0.25) (layer B.Cu) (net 2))
 (segment (start 146.05 109.22) (end 146.05 102.87) (width 0.25) (layer B.Cu) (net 2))
 (segment (start 149.78 95.47) (end 146.27 95.47) (width 0.25) (layer B.Cu) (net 2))
 (segment (start 146.27 95.47) (end 146.05 95.25) (width 0.25) (layer B.Cu) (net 2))
 (segment (start 146.05 102.87) (end 146.05 95.25) (width 0.25) (layer B.Cu) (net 2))
 (segment (start 146.89 88.47) (end 146.05 87.63) (width 0.25) (layer B.Cu) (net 2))
 (segment (start 149.78 88.47) (end 146.89 88.47) (width 0.25) (layer B.Cu) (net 2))
 (segment (start 146.05 95.25) (end 146.05 87.63) (width 0.25) (layer B.Cu) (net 2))
 (segment (start 146.24 81.47) (end 146.05 81.28) (width 0.25) (layer B.Cu) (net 2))
 (segment (start 149.78 81.47) (end 146.24 81.47) (width 0.25) (layer B.Cu) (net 2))
 (segment (start 146.05 87.63) (end 146.05 81.28) (width 0.25) (layer B.Cu) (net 2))
 (segment (start 146.05 81.28) (end 146.05 74.93) (width 0.25) (layer B.Cu) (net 2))
 (segment (start 127 137.16) (end 127 140.97) (width 0.25) (layer B.Cu) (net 2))
 (segment (start 127 134.62) (end 127 137.16) (width 0.25) (layer B.Cu) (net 2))
 (segment (start 142.86 140.97) (end 146.36 137.47) (width 0.25) (layer B.Cu) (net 2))
 (segment (start 127 140.97) (end 142.86 140.97) (width 0.25) (layer B.Cu) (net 2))
 (segment (start 141 77.5) (end 143.57 74.93) (width 0.25) (layer B.Cu) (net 2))
 (segment (start 146.05 74.93) (end 143.57 74.93) (width 0.25) (layer B.Cu) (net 2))
 (segment (start 143.57 74.93) (end 143.51 74.93) (width 0.25) (layer B.Cu) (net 2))
 (segment (start 134.62 83.5) (end 131 83.5) (width 0.25) (layer F.Cu) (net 1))
 (segment (start 130.84 83.34) (end 130.84 77.5) (width 0.25) (layer F.Cu) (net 1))
 (segment (start 131 83.5) (end 130.84 83.34) (width 0.25) (layer F.Cu) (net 1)))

